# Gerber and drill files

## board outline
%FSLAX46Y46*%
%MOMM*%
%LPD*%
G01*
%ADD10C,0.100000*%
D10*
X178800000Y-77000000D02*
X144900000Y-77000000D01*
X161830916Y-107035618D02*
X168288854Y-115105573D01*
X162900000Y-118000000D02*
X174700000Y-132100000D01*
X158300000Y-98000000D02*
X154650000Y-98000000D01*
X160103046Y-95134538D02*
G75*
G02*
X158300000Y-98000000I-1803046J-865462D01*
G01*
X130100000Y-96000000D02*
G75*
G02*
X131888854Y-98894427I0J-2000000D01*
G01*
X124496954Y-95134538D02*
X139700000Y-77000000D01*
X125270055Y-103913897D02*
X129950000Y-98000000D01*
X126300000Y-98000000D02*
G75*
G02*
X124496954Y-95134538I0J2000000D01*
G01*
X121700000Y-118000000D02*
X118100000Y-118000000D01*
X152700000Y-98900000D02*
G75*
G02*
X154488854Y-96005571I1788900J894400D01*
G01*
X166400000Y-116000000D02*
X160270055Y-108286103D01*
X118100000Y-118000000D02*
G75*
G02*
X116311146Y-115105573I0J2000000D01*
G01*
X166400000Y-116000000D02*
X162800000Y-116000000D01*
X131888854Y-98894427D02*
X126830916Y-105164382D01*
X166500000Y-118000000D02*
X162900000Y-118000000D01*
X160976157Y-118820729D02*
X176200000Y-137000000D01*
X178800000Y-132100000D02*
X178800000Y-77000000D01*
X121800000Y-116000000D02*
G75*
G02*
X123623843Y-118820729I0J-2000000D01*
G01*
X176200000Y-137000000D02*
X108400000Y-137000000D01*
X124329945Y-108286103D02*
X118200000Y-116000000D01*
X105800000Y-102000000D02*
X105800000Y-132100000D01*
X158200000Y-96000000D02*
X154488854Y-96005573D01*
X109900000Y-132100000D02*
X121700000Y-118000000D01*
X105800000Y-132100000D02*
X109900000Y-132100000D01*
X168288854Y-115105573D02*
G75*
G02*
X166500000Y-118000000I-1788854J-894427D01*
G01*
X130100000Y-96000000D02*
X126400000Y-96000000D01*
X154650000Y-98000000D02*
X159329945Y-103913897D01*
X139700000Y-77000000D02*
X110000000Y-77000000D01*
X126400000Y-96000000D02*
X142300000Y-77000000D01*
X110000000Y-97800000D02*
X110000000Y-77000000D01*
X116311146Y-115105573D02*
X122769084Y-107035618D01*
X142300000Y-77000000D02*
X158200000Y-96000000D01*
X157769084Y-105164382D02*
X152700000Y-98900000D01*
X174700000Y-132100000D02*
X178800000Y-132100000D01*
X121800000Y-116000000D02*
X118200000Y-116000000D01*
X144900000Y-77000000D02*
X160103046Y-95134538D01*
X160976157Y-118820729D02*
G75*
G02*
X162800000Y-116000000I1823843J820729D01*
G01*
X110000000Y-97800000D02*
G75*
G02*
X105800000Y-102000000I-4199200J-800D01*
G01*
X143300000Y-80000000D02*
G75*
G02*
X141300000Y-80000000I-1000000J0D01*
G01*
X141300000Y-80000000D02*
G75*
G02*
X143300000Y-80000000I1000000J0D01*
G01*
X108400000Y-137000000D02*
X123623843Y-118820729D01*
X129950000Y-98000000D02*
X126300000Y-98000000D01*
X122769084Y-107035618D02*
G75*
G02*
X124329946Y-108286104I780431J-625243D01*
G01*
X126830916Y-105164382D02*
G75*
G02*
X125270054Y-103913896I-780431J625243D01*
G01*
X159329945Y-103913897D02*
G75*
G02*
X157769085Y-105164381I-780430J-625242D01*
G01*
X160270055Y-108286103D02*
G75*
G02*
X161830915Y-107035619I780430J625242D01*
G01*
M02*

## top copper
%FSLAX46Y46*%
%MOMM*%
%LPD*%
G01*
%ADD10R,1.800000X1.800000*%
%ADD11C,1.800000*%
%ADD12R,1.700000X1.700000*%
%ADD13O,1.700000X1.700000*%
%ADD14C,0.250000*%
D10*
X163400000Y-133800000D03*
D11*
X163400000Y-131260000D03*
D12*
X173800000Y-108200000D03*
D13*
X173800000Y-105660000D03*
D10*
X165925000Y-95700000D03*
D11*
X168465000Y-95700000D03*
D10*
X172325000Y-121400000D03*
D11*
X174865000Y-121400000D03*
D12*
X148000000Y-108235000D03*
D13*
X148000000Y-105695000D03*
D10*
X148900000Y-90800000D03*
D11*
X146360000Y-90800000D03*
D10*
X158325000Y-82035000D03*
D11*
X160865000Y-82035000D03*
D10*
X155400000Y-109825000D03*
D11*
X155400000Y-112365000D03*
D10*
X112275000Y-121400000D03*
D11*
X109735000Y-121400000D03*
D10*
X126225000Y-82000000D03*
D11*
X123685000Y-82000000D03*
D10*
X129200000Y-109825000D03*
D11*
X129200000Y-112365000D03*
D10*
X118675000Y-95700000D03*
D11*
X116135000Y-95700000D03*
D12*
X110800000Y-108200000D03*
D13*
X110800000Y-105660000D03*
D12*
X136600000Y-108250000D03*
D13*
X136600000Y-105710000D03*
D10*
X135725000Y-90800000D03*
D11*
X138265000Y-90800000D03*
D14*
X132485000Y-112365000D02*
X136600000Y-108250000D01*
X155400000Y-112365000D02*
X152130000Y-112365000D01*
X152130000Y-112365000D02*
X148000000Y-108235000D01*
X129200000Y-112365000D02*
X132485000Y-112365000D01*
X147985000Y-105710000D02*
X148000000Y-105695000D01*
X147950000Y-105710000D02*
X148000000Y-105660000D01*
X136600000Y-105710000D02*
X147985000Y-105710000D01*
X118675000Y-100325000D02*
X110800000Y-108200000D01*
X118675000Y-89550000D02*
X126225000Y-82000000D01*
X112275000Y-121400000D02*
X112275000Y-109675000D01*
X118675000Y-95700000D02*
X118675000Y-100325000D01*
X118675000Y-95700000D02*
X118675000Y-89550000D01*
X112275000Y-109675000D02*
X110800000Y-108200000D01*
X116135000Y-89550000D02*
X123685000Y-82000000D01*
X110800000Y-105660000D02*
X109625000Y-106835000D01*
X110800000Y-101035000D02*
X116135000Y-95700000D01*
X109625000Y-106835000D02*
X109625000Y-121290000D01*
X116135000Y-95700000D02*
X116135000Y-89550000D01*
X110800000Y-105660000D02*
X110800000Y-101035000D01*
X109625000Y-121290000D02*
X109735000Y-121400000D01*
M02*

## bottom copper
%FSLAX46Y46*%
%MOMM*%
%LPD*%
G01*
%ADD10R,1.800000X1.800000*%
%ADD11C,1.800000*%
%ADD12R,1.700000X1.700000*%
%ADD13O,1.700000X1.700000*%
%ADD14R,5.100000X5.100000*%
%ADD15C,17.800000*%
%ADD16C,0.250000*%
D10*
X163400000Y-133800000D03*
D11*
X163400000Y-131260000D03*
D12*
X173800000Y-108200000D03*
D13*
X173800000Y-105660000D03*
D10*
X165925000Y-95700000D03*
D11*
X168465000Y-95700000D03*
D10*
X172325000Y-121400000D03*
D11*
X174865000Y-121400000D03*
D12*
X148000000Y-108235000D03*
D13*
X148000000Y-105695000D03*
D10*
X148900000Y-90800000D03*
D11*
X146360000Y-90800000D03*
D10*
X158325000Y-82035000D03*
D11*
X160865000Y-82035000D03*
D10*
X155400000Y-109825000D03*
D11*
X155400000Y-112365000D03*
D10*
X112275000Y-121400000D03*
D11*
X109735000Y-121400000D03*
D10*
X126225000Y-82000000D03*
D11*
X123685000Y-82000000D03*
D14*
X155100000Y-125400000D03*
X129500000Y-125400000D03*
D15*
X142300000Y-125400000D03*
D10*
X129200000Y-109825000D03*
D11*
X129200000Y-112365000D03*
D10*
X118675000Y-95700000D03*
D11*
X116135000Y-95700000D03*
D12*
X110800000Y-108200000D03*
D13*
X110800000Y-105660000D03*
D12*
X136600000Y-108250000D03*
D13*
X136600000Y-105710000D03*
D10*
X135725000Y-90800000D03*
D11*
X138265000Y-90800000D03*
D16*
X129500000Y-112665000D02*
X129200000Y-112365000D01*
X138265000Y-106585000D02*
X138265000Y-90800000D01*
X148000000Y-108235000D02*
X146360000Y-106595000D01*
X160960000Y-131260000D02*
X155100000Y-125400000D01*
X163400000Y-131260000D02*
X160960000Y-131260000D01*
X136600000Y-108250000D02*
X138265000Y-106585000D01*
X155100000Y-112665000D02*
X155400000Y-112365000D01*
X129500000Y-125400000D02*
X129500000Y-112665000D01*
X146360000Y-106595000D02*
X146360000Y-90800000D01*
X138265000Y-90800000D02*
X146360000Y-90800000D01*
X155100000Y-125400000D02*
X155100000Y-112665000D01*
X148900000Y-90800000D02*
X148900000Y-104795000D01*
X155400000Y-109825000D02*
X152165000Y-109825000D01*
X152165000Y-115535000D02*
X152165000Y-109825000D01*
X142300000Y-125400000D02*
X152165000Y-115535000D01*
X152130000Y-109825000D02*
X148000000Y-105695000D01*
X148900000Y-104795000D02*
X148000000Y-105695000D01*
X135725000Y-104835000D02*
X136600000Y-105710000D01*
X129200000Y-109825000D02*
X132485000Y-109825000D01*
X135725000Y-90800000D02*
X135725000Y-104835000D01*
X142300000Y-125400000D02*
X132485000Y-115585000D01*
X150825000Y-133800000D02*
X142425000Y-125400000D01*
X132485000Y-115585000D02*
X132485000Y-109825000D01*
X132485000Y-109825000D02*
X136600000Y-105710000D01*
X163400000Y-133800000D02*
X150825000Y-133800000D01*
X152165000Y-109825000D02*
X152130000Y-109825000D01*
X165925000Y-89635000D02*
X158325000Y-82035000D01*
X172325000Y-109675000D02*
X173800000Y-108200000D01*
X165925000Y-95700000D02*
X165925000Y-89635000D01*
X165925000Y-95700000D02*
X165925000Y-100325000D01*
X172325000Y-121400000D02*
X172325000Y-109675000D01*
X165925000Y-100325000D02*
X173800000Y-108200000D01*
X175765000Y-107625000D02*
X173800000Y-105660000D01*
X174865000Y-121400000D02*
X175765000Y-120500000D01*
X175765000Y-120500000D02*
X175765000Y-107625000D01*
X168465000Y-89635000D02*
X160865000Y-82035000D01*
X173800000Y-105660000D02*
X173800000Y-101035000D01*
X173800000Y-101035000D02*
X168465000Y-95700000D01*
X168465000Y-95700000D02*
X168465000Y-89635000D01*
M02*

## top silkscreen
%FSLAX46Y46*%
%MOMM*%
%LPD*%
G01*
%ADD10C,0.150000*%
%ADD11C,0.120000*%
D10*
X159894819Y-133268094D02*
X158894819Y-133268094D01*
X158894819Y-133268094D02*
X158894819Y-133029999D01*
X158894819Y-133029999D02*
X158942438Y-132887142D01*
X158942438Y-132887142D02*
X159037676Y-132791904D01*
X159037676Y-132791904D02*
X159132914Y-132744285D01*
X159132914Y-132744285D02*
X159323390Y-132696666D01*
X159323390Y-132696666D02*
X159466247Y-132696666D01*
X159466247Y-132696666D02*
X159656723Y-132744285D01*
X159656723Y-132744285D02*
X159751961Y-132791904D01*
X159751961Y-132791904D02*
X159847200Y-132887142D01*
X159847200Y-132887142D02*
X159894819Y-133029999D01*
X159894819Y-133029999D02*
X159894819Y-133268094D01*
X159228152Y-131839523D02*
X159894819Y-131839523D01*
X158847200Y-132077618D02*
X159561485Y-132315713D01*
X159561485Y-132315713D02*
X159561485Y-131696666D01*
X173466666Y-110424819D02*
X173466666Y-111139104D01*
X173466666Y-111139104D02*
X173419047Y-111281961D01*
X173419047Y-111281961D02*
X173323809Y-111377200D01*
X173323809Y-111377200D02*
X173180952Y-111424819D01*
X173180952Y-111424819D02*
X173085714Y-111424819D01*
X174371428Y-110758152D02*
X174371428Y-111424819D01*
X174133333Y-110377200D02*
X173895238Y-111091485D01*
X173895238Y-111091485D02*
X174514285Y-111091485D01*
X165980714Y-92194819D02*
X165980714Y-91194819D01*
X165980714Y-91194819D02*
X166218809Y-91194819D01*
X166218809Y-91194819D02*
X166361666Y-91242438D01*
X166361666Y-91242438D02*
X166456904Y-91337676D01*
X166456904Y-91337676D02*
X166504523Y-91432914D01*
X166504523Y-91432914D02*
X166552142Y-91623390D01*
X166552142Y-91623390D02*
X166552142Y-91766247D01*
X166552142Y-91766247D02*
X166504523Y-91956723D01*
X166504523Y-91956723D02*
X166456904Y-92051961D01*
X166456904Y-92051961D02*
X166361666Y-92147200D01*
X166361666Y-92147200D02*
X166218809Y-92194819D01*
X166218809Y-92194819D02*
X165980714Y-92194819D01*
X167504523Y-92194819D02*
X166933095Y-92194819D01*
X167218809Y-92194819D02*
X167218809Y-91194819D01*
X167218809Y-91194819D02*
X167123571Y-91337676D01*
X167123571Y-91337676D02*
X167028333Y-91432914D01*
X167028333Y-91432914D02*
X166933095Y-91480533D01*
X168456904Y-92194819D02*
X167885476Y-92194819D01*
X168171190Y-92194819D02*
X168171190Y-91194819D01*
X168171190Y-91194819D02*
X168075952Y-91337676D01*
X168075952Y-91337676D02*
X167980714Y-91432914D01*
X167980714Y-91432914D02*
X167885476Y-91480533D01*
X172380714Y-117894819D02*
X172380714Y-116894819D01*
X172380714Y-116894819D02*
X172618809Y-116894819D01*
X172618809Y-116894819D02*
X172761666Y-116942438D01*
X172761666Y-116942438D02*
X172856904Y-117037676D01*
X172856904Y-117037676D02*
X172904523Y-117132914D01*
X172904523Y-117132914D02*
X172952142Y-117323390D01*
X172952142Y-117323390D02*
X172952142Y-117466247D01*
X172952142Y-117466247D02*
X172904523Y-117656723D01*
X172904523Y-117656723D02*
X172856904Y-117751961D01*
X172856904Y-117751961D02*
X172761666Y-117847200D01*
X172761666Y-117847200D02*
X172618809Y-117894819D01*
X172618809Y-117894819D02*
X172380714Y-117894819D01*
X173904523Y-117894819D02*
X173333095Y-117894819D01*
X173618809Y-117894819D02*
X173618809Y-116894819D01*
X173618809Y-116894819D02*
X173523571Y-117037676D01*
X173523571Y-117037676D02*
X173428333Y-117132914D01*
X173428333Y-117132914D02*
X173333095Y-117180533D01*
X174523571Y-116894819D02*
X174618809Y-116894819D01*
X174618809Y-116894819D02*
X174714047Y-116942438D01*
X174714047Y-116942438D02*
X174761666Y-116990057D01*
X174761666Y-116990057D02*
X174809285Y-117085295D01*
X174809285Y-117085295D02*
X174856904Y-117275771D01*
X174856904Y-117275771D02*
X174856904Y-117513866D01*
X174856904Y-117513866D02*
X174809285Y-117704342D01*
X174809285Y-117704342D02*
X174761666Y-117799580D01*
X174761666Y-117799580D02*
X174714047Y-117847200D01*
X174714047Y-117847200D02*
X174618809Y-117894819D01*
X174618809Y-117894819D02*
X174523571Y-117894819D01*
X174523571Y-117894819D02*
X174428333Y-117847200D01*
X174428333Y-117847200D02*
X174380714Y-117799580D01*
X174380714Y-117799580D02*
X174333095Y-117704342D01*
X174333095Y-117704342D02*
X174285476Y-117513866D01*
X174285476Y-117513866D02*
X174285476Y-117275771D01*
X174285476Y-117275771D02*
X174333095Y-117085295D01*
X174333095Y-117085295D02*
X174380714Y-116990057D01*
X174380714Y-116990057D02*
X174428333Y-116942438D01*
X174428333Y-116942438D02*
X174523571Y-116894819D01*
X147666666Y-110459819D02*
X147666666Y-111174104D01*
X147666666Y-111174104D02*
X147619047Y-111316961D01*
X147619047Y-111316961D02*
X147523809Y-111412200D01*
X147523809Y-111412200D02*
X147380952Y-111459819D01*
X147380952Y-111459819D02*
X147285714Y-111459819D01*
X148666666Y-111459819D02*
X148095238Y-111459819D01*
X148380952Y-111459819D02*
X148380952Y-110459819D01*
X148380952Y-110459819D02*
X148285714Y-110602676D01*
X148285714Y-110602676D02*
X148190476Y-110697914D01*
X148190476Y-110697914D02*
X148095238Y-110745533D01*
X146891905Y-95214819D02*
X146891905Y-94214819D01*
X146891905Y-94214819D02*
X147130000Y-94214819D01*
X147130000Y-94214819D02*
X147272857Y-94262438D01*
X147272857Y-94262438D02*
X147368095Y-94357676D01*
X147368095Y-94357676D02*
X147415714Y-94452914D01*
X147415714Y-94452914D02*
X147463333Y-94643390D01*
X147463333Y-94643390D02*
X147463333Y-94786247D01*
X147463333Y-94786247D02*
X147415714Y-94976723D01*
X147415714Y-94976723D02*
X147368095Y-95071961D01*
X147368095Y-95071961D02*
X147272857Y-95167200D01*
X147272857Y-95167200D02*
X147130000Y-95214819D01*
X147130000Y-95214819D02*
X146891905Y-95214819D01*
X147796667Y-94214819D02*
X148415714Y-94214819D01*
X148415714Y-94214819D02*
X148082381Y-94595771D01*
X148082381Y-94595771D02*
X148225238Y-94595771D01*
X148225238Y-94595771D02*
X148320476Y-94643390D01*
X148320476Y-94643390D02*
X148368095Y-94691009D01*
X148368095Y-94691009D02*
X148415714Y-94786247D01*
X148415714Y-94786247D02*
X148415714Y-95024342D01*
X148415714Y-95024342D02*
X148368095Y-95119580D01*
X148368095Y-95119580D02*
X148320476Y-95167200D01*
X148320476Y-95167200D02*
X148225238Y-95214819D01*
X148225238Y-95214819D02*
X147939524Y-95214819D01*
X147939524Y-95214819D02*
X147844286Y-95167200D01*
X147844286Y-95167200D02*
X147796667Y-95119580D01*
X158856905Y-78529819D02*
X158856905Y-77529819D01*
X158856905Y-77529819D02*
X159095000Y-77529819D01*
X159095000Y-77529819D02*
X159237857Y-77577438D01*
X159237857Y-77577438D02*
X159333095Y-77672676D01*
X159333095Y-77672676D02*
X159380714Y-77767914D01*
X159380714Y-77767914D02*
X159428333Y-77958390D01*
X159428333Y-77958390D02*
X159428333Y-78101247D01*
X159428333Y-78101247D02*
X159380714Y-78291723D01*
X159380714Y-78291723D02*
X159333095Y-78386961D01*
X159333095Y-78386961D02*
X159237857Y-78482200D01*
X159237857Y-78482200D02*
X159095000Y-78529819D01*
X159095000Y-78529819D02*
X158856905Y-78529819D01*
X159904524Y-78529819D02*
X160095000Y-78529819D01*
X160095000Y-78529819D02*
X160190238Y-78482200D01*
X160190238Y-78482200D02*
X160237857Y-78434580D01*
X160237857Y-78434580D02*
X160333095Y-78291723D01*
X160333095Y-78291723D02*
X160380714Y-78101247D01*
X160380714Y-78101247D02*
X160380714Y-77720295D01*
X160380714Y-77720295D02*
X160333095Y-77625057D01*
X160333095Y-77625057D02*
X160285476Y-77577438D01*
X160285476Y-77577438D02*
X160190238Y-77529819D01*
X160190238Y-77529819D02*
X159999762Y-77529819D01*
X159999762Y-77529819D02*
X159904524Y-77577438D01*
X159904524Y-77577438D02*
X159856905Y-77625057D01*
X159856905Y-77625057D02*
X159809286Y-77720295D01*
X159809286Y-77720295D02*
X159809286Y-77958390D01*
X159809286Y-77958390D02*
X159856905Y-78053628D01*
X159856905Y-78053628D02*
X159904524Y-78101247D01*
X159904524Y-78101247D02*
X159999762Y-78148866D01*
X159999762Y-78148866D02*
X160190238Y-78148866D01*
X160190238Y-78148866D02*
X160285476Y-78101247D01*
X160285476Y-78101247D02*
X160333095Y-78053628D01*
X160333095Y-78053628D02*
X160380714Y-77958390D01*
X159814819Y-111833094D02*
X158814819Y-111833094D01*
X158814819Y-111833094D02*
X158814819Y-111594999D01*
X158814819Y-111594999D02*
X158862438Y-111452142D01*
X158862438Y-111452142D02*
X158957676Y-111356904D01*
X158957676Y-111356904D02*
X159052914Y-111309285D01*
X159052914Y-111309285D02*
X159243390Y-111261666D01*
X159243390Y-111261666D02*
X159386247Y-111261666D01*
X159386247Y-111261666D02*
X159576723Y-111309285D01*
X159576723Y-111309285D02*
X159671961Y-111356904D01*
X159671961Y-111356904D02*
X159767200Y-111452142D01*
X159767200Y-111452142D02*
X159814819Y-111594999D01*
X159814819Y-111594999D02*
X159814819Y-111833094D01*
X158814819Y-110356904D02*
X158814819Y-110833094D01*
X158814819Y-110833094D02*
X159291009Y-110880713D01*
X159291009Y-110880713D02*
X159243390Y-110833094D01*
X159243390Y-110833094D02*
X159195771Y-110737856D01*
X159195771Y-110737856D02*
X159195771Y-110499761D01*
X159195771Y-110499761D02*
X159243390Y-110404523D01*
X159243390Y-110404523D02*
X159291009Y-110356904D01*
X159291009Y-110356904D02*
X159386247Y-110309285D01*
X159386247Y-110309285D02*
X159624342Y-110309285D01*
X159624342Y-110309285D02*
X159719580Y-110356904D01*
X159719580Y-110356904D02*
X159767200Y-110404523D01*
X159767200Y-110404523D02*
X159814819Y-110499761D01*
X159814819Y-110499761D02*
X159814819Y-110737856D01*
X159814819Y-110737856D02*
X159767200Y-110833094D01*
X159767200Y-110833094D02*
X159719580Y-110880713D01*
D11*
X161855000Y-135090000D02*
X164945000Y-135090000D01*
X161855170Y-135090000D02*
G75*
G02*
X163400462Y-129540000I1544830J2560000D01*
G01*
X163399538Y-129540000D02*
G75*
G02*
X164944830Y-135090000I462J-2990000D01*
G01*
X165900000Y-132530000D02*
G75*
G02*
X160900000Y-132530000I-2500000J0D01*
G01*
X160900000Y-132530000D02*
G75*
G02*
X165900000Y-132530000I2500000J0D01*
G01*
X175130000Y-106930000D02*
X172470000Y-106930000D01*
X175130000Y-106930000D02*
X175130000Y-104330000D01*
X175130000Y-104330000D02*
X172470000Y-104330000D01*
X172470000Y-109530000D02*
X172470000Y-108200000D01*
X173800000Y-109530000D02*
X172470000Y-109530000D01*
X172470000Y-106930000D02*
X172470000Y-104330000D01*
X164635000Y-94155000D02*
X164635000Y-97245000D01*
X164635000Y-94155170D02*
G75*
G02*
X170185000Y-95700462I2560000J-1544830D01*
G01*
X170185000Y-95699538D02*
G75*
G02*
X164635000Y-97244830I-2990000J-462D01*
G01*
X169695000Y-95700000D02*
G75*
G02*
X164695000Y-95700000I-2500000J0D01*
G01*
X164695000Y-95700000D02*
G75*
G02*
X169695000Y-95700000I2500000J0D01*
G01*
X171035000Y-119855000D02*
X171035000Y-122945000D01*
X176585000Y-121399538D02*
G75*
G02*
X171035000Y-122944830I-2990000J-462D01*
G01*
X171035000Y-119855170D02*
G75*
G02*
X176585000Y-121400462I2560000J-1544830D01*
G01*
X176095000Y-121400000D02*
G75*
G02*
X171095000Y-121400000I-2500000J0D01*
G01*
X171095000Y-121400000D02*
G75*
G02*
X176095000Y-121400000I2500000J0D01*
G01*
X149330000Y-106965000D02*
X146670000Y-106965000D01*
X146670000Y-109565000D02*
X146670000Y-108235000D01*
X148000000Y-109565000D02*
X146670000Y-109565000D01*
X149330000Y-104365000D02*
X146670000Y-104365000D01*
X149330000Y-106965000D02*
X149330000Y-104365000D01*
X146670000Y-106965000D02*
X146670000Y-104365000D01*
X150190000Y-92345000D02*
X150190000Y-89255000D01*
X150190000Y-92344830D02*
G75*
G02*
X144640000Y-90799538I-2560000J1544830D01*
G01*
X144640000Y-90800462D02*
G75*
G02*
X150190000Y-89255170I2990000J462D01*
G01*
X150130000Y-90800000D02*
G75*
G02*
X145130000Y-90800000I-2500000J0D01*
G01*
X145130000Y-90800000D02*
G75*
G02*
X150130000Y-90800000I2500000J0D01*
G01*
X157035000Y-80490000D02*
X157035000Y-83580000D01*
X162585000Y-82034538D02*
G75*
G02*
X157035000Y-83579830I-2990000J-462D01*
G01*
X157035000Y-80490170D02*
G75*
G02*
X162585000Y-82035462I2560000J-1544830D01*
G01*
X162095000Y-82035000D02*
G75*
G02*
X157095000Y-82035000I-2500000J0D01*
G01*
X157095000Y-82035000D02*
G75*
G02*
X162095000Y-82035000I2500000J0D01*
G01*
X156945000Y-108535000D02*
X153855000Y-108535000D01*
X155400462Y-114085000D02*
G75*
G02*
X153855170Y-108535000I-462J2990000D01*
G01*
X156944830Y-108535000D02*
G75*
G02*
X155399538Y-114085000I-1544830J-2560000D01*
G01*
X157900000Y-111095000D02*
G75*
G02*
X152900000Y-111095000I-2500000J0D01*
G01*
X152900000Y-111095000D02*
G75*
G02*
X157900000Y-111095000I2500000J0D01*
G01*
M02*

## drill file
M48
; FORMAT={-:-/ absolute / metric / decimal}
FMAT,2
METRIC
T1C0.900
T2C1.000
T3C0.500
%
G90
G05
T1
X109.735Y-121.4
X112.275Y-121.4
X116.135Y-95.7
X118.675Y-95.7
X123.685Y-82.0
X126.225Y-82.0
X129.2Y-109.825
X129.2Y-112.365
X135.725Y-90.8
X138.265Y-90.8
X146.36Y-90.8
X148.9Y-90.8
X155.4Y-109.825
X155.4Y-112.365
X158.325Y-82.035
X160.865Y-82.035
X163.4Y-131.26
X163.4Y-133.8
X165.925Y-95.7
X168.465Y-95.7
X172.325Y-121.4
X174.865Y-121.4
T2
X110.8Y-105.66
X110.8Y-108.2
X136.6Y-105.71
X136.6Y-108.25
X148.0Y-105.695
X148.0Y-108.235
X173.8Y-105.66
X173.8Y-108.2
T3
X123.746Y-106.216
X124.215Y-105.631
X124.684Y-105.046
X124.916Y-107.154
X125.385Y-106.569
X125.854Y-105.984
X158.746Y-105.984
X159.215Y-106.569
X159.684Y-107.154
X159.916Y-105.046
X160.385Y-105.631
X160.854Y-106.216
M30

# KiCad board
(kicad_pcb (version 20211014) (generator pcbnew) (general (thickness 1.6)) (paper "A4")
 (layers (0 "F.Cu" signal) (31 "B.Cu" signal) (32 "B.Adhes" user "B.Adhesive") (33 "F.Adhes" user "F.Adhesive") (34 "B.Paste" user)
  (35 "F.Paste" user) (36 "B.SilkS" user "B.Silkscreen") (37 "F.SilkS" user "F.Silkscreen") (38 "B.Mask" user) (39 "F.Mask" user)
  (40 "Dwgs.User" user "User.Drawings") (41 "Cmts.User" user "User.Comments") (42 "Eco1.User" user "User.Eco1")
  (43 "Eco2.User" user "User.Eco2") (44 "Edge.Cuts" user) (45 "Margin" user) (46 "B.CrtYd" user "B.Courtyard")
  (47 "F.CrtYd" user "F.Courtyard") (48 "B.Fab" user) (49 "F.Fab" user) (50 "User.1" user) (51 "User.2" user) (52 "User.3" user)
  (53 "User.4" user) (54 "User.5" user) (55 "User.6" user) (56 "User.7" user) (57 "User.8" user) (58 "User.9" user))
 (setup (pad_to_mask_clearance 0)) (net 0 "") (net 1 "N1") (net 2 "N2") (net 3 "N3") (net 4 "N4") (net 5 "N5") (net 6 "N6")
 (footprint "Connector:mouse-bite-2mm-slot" (layer "F.Cu") (at 124.8 106.1 -128.7)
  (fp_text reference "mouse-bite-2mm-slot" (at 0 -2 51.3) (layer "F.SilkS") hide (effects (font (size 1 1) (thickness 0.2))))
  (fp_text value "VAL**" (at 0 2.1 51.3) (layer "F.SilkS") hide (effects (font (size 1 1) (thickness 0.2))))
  (fp_arc (start 2 1) (mid 1 0) (end 2 -1) (layer "Edge.Cuts") (width 0.1))
  (fp_arc (start -2 -1) (mid -1 0) (end -2 1) (layer "Edge.Cuts") (width 0.1))
  (pad "" np_thru_hole circle (at 0.75 0.75 231.3) (size 0.5 0.5) (drill 0.5) (layers F&B.Cu *.Mask))
  (pad "" np_thru_hole circle (at 0.75 -0.75 231.3) (size 0.5 0.5) (drill 0.5) (layers F&B.Cu *.Mask))
  (pad "" np_thru_hole circle (at 0 0.75 231.3) (size 0.5 0.5) (drill 0.5) (layers F&B.Cu *.Mask))
  (pad "" np_thru_hole circle (at 0 -0.75 231.3) (size 0.5 0.5) (drill 0.5) (layers F&B.Cu *.Mask))
  (pad "" np_thru_hole circle (at -0.75 0.75 231.3) (size 0.5 0.5) (drill 0.5) (layers F&B.Cu *.Mask))
  (pad "" np_thru_hole circle (at -0.75 -0.75 231.3) (size 0.5 0.5) (drill 0.5) (layers F&B.Cu *.Mask)))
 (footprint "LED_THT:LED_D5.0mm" (layer "F.Cu") (at 163.4 133.8 90)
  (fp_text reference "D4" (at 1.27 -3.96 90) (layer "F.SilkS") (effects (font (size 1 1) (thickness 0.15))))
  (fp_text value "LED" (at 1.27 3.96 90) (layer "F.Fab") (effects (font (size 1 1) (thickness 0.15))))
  (fp_line (start -1.29 -1.545) (end -1.29 1.545) (layer "F.SilkS") (width 0.12))
  (fp_arc (start -1.29 -1.54483) (mid 2.072002 -2.880433) (end 4.26 0.000462) (layer "F.SilkS") (width 0.12))
  (fp_arc (start 4.26 -0.000462) (mid 2.072002 2.880433) (end -1.29 1.54483) (layer "F.SilkS") (width 0.12))
  (fp_circle (center 1.27 0) (end 3.77 0) (layer "F.SilkS") (width 0.12) (fill none))
  (pad "1" thru_hole rect (at 0 0 90) (size 1.8 1.8) (drill 0.9) (layers *.Cu *.Mask) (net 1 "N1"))
  (pad "2" thru_hole circle (at 2.54 0 90) (size 1.8 1.8) (drill 0.9) (layers *.Cu *.Mask) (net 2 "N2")))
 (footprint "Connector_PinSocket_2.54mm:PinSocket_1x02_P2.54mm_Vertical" (layer "F.Cu") (at 173.8 108.2 180)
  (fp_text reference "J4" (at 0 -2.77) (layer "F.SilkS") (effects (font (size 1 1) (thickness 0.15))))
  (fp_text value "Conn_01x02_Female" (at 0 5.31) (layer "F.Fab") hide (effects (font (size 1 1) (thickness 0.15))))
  (fp_line (start -1.33 1.27) (end 1.33 1.27) (layer "F.SilkS") (width 0.12))
  (fp_line (start -1.33 1.27) (end -1.33 3.87) (layer "F.SilkS") (width 0.12))
  (fp_line (start -1.33 3.87) (end 1.33 3.87) (layer "F.SilkS") (width 0.12))
  (fp_line (start 1.33 -1.33) (end 1.33 0) (layer "F.SilkS") (width 0.12))
  (fp_line (start 0 -1.33) (end 1.33 -1.33) (layer "F.SilkS") (width 0.12))
  (fp_line (start 1.33 1.27) (end 1.33 3.87) (layer "F.SilkS") (width 0.12))
  (pad "1" thru_hole rect (at 0 0 180) (size 1.7 1.7) (drill 1) (layers *.Cu *.Mask) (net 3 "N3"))
  (pad "2" thru_hole oval (at 0 2.54 180) (size 1.7 1.7) (drill 1) (layers *.Cu *.Mask) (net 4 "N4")))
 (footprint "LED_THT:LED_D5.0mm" (layer "F.Cu") (at 165.925 95.7)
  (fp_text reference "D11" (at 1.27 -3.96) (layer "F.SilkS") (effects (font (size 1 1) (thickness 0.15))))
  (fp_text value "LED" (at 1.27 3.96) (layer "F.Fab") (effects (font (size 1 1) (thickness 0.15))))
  (fp_line (start -1.29 -1.545) (end -1.29 1.545) (layer "F.SilkS") (width 0.12))
  (fp_arc (start -1.29 -1.54483) (mid 2.072002 -2.880433) (end 4.26 0.000462) (layer "F.SilkS") (width 0.12))
  (fp_arc (start 4.26 -0.000462) (mid 2.072002 2.880433) (end -1.29 1.54483) (layer "F.SilkS") (width 0.12))
  (fp_circle (center 1.27 0) (end 3.77 0) (layer "F.SilkS") (width 0.12) (fill none))
  (pad "1" thru_hole rect (at 0 0) (size 1.8 1.8) (drill 0.9) (layers *.Cu *.Mask) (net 3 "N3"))
  (pad "2" thru_hole circle (at 2.54 0) (size 1.8 1.8) (drill 0.9) (layers *.Cu *.Mask) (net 4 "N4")))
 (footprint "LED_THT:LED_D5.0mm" (layer "F.Cu") (at 172.325 121.4)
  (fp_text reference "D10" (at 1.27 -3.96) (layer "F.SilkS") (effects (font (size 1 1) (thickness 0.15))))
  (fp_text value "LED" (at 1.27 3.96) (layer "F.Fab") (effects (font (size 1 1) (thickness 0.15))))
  (fp_line (start -1.29 -1.545) (end -1.29 1.545) (layer "F.SilkS") (width 0.12))
  (fp_arc (start 4.26 -0.000462) (mid 2.072002 2.880433) (end -1.29 1.54483) (layer "F.SilkS") (width 0.12))
  (fp_arc (start -1.29 -1.54483) (mid 2.072002 -2.880433) (end 4.26 0.000462) (layer "F.SilkS") (width 0.12))
  (fp_circle (center 1.27 0) (end 3.77 0) (layer "F.SilkS") (width 0.12) (fill none))
  (pad "1" thru_hole rect (at 0 0) (size 1.8 1.8) (drill 0.9) (layers *.Cu *.Mask) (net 3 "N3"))
  (pad "2" thru_hole circle (at 2.54 0) (size 1.8 1.8) (drill 0.9) (layers *.Cu *.Mask) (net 4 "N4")))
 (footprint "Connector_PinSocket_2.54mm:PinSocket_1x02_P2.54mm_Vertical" (layer "F.Cu") (at 148 108.235 180)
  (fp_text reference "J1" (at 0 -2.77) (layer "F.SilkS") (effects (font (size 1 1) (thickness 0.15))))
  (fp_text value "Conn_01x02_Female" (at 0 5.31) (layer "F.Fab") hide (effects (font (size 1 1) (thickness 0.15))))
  (fp_line (start -1.33 1.27) (end 1.33 1.27) (layer "F.SilkS") (width 0.12))
  (fp_line (start 1.33 -1.33) (end 1.33 0) (layer "F.SilkS") (width 0.12))
  (fp_line (start 0 -1.33) (end 1.33 -1.33) (layer "F.SilkS") (width 0.12))
  (fp_line (start -1.33 3.87) (end 1.33 3.87) (layer "F.SilkS") (width 0.12))
  (fp_line (start -1.33 1.27) (end -1.33 3.87) (layer "F.SilkS") (width 0.12))
  (fp_line (start 1.33 1.27) (end 1.33 3.87) (layer "F.SilkS") (width 0.12))
  (pad "1" thru_hole rect (at 0 0 180) (size 1.7 1.7) (drill 1) (layers *.Cu *.Mask) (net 2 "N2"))
  (pad "2" thru_hole oval (at 0 2.54 180) (size 1.7 1.7) (drill 1) (layers *.Cu *.Mask) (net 1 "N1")))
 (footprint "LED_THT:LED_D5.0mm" (layer "F.Cu") (at 148.9 90.8 180)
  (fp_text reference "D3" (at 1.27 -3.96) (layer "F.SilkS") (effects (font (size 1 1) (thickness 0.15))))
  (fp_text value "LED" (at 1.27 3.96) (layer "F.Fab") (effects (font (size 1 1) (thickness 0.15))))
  (fp_line (start -1.29 -1.545) (end -1.29 1.545) (layer "F.SilkS") (width 0.12))
  (fp_arc (start -1.29 -1.54483) (mid 2.072002 -2.880433) (end 4.26 0.000462) (layer "F.SilkS") (width 0.12))
  (fp_arc (start 4.26 -0.000462) (mid 2.072002 2.880433) (end -1.29 1.54483) (layer "F.SilkS") (width 0.12))
  (fp_circle (center 1.27 0) (end 3.77 0) (layer "F.SilkS") (width 0.12) (fill none))
  (pad "1" thru_hole rect (at 0 0 180) (size 1.8 1.8) (drill 0.9) (layers *.Cu *.Mask) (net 1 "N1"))
  (pad "2" thru_hole circle (at 2.54 0 180) (size 1.8 1.8) (drill 0.9) (layers *.Cu *.Mask) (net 2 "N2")))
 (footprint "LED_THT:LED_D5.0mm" (layer "F.Cu") (at 158.325 82.035)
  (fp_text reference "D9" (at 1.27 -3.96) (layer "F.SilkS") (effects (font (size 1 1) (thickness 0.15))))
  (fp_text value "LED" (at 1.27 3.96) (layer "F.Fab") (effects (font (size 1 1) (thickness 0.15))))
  (fp_line (start -1.29 -1.545) (end -1.29 1.545) (layer "F.SilkS") (width 0.12))
  (fp_arc (start 4.26 -0.000462) (mid 2.072002 2.880433) (end -1.29 1.54483) (layer "F.SilkS") (width 0.12))
  (fp_arc (start -1.29 -1.54483) (mid 2.072002 -2.880433) (end 4.26 0.000462) (layer "F.SilkS") (width 0.12))
  (fp_circle (center 1.27 0) (end 3.77 0) (layer "F.SilkS") (width 0.12) (fill none))
  (pad "1" thru_hole rect (at 0 0) (size 1.8 1.8) (drill 0.9) (layers *.Cu *.Mask) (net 3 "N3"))
  (pad "2" thru_hole circle (at 2.54 0) (size 1.8 1.8) (drill 0.9) (layers *.Cu *.Mask) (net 4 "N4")))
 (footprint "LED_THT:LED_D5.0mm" (layer "F.Cu") (at 155.4 109.825 -90)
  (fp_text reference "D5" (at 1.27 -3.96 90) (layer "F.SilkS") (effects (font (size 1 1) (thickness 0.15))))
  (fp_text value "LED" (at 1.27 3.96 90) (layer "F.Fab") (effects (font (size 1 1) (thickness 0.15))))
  (fp_line (start -1.29 -1.545) (end -1.29 1.545) (layer "F.SilkS") (width 0.12))
  (fp_arc (start 4.26 -0.000462) (mid 2.072002 2.880433) (end -1.29 1.54483) (layer "F.SilkS") (width 0.12))
  (fp_arc (start -1.29 -1.54483) (mid 2.072002 -2.880433) (end 4.26 0.000462) (layer "F.SilkS") (width 0.12))
  (fp_circle (center 1.27 0) (end 3.77 0) (layer "F.SilkS") (width 0.12) (fill none))
  (pad "1" thru_hole rect (at 0 0 270) (size 1.8 1.8) (drill 0.9) (layers *.Cu *.Mask) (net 1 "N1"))
  (pad "2" thru_hole circle (at 2.54 0 270) (size 1.8 1.8) (drill 0.9) (layers *.Cu *.Mask) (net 2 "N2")))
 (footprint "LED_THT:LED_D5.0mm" (layer "B.Cu") (at 112.275 121.4 180)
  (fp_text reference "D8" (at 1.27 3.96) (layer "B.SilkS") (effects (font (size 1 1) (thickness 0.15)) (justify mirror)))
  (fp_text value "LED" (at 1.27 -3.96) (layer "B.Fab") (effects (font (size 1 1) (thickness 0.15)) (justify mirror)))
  (pad "1" thru_hole rect (at 0 0 180) (size 1.8 1.8) (drill 0.9) (layers *.Cu *.Mask) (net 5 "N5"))
  (pad "2" thru_hole circle (at 2.54 0 180) (size 1.8 1.8) (drill 0.9) (layers *.Cu *.Mask) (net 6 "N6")))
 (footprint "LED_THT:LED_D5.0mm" (layer "B.Cu") (at 126.225 82 180)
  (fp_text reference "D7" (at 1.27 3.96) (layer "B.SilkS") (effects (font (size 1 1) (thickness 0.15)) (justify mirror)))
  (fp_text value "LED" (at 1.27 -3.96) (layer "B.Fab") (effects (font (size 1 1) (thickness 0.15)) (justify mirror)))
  (pad "1" thru_hole rect (at 0 0 180) (size 1.8 1.8) (drill 0.9) (layers *.Cu *.Mask) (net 5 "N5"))
  (pad "2" thru_hole circle (at 2.54 0 180) (size 1.8 1.8) (drill 0.9) (layers *.Cu *.Mask) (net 6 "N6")))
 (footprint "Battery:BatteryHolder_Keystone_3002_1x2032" (layer "B.Cu") (at 142.3 125.4)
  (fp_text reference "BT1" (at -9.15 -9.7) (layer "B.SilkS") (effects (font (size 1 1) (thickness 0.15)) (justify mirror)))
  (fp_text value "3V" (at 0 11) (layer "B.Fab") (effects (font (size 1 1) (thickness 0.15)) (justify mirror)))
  (pad "1" smd rect (at 12.8 0) (size 5.1 5.1) (layers "B.Cu" "B.Paste" "B.Mask") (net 2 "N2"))
  (pad "1" smd rect (at -12.8 0) (size 5.1 5.1) (layers "B.Cu" "B.Paste" "B.Mask") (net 2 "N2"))
  (pad "2" smd circle (at 0 0) (size 17.8 17.8) (layers "B.Cu" "B.Mask") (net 1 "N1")))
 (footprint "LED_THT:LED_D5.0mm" (layer "B.Cu") (at 129.2 109.825 -90)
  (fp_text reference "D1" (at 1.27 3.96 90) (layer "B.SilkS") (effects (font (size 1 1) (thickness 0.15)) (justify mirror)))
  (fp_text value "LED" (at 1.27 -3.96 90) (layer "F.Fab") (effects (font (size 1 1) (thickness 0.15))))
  (pad "1" thru_hole rect (at 0 0 270) (size 1.8 1.8) (drill 0.9) (layers *.Cu *.Mask) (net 1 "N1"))
  (pad "2" thru_hole circle (at 2.54 0 270) (size 1.8 1.8) (drill 0.9) (layers *.Cu *.Mask) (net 2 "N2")))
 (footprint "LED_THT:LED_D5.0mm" (layer "B.Cu") (at 118.675 95.7 180)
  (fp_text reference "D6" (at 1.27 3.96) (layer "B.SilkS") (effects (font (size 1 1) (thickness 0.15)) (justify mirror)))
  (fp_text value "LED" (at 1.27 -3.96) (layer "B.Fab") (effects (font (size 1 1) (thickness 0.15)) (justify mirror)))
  (pad "1" thru_hole rect (at 0 0 180) (size 1.8 1.8) (drill 0.9) (layers *.Cu *.Mask) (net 5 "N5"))
  (pad "2" thru_hole circle (at 2.54 0 180) (size 1.8 1.8) (drill 0.9) (layers *.Cu *.Mask) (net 6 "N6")))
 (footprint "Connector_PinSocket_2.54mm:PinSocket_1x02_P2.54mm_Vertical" (layer "B.Cu") (at 110.8 108.2)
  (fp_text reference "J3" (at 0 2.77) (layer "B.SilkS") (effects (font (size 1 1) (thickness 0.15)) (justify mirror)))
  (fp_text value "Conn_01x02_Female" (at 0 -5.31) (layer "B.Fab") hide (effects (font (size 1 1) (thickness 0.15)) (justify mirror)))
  (pad "1" thru_hole rect locked (at 0 0) (size 1.7 1.7) (drill 1) (layers *.Cu *.Mask) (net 5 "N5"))
  (pad "2" thru_hole oval (at 0 -2.54) (size 1.7 1.7) (drill 1) (layers *.Cu *.Mask) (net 6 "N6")))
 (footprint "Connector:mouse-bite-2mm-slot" (layer "B.Cu") (at 159.8 106.1 -51.3)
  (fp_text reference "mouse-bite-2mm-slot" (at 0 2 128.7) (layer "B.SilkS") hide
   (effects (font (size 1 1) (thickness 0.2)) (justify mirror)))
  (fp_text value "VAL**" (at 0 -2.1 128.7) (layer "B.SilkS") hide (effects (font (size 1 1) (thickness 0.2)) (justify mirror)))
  (fp_arc (start -2 -1) (mid -1 0) (end -2 1) (layer "Edge.Cuts") (width 0.1))
  (fp_arc (start 2 1) (mid 1 0) (end 2 -1) (layer "Edge.Cuts") (width 0.1))
  (pad "" np_thru_hole circle (at 0.75 -0.75 308.7) (size 0.5 0.5) (drill 0.5) (layers *.Cu *.Mask))
  (pad "" np_thru_hole circle (at 0 0.75 308.7) (size 0.5 0.5) (drill 0.5) (layers *.Cu *.Mask))
  (pad "" np_thru_hole circle (at -0.75 0.75 308.7) (size 0.5 0.5) (drill 0.5) (layers *.Cu *.Mask))
  (pad "" np_thru_hole circle (at 0 -0.75 308.7) (size 0.5 0.5) (drill 0.5) (layers *.Cu *.Mask))
  (pad "" np_thru_hole circle (at 0.75 0.75 308.7) (size 0.5 0.5) (drill 0.5) (layers *.Cu *.Mask))
  (pad "" np_thru_hole circle (at -0.75 -0.75 308.7) (size 0.5 0.5) (drill 0.5) (layers *.Cu *.Mask)))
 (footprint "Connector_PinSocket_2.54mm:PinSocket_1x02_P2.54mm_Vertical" (layer "B.Cu") (at 136.6 108.25)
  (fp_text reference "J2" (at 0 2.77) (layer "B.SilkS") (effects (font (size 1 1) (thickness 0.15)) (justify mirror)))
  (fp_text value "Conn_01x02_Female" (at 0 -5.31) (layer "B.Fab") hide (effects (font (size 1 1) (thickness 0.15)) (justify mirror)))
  (pad "1" thru_hole rect (at 0 0) (size 1.7 1.7) (drill 1) (layers *.Cu *.Mask) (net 2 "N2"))
  (pad "2" thru_hole oval (at 0 -2.54) (size 1.7 1.7) (drill 1) (layers *.Cu *.Mask) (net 1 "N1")))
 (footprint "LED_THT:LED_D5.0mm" (layer "B.Cu") (at 135.725 90.8)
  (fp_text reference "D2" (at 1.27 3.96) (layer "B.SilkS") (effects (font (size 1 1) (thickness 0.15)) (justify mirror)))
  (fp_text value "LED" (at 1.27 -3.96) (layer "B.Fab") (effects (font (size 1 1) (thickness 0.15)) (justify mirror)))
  (pad "1" thru_hole rect (at 0 0) (size 1.8 1.8) (drill 0.9) (layers *.Cu *.Mask) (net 1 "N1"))
  (pad "2" thru_hole circle (at 2.54 0) (size 1.8 1.8) (drill 0.9) (layers *.Cu *.Mask) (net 2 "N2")))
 (gr_line (start 178.8 77) (end 144.9 77) (layer "Edge.Cuts") (width 0.1))
 (gr_line (start 161.830916 107.035618) (end 168.288854 115.105573) (layer "Edge.Cuts") (width 0.1))
 (gr_line (start 162.9 118) (end 174.7 132.1) (layer "Edge.Cuts") (width 0.1))
 (gr_line (start 158.3 98) (end 154.65 98) (layer "Edge.Cuts") (width 0.1))
 (gr_arc (start 160.103046 95.134538) (mid 159.992767 97.065147) (end 158.3 98) (layer "Edge.Cuts") (width 0.1))
 (gr_arc (start 130.1 96) (mid 131.801302 96.948538) (end 131.888854 98.894427) (layer "Edge.Cuts") (width 0.1))
 (gr_line (start 124.496954 95.134538) (end 139.7 77) (layer "Edge.Cuts") (width 0.1))
 (gr_line (start 125.270055 103.913897) (end 129.95 98) (layer "Edge.Cuts") (width 0.1))
 (gr_arc (start 126.3 98) (mid 124.607232 97.065147) (end 124.496954 95.134538) (layer "Edge.Cuts") (width 0.1))
 (gr_line (start 121.7 118) (end 118.1 118) (layer "Edge.Cuts") (width 0.1))
 (gr_arc (start 152.7 98.9) (mid 152.787574 96.954123) (end 154.488854 96.005573) (layer "Edge.Cuts") (width 0.1))
 (gr_line (start 166.4 116) (end 160.270055 108.286103) (layer "Edge.Cuts") (width 0.1))
 (gr_arc (start 118.1 118) (mid 116.398698 117.051462) (end 116.311146 115.105573) (layer "Edge.Cuts") (width 0.1))
 (gr_line (start 166.4 116) (end 162.8 116) (layer "Edge.Cuts") (width 0.1))
 (gr_line (start 131.888854 98.894427) (end 126.830916 105.164382) (layer "Edge.Cuts") (width 0.1))
 (gr_line (start 166.5 118) (end 162.9 118) (layer "Edge.Cuts") (width 0.1))
 (gr_line (start 160.976157 118.820729) (end 176.2 137) (layer "Edge.Cuts") (width 0.1))
 (gr_line (start 178.8 132.1) (end 178.8 77) (layer "Edge.Cuts") (width 0.1))
 (gr_arc (start 121.8 116) (mid 123.479503 116.914058) (end 123.623843 118.820729) (layer "Edge.Cuts") (width 0.1))
 (gr_line (start 176.2 137) (end 108.4 137) (layer "Edge.Cuts") (width 0.1))
 (gr_line (start 124.329945 108.286103) (end 118.2 116) (layer "Edge.Cuts") (width 0.1))
 (gr_line (start 105.8 102) (end 105.8 132.1) (layer "Edge.Cuts") (width 0.1))
 (gr_line (start 158.2 96) (end 154.488854 96.005573) (layer "Edge.Cuts") (width 0.1))
 (gr_line (start 109.9 132.1) (end 121.7 118) (layer "Edge.Cuts") (width 0.1))
 (gr_line (start 105.8 132.1) (end 109.9 132.1) (layer "Edge.Cuts") (width 0.1))
 (gr_arc (start 168.288854 115.105573) (mid 168.201301 117.051462) (end 166.5 118) (layer "Edge.Cuts") (width 0.1))
 (gr_line (start 130.1 96) (end 126.4 96) (layer "Edge.Cuts") (width 0.1))
 (gr_line (start 154.65 98) (end 159.329945 103.913897) (layer "Edge.Cuts") (width 0.1))
 (gr_line (start 139.7 77) (end 110 77) (layer "Edge.Cuts") (width 0.1))
 (gr_line (start 126.4 96) (end 142.3 77) (layer "Edge.Cuts") (width 0.1))
 (gr_line (start 110 97.8) (end 110 77) (layer "Edge.Cuts") (width 0.1))
 (gr_line (start 116.311146 115.105573) (end 122.769084 107.035618) (layer "Edge.Cuts") (width 0.1))
 (gr_line (start 142.3 77) (end 158.2 96) (layer "Edge.Cuts") (width 0.1))
 (gr_line (start 157.769084 105.164382) (end 152.7 98.9) (layer "Edge.Cuts") (width 0.1))
 (gr_line (start 174.7 132.1) (end 178.8 132.1) (layer "Edge.Cuts") (width 0.1))
 (gr_line (start 121.8 116) (end 118.2 116) (layer "Edge.Cuts") (width 0.1))
 (gr_line (start 144.9 77) (end 160.103046 95.134538) (layer "Edge.Cuts") (width 0.1))
 (gr_arc (start 160.976157 118.820729) (mid 161.120498 116.914058) (end 162.8 116) (layer "Edge.Cuts") (width 0.1))
 (gr_arc (start 110 97.8) (mid 108.770083 100.770083) (end 105.8 102) (layer "Edge.Cuts") (width 0.1))
 (gr_circle (center 142.3 80) (end 142.3 81) (layer "Edge.Cuts") (width 0.1) (fill none))
 (gr_line (start 108.4 137) (end 123.623843 118.820729) (layer "Edge.Cuts") (width 0.1))
 (gr_line (start 129.95 98) (end 126.3 98) (layer "Edge.Cuts") (width 0.1))
 (segment (start 132.485 112.365) (end 136.6 108.25) (width 0.25) (layer "F.Cu") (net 2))
 (segment (start 155.4 112.365) (end 152.13 112.365) (width 0.25) (layer "F.Cu") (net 2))
 (segment (start 152.13 112.365) (end 148 108.235) (width 0.25) (layer "F.Cu") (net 2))
 (segment (start 129.2 112.365) (end 132.485 112.365) (width 0.25) (layer "F.Cu") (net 2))
 (segment (start 129.5 112.665) (end 129.2 112.365) (width 0.25) (layer "B.Cu") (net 2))
 (segment (start 138.265 106.585) (end 138.265 90.8) (width 0.25) (layer "B.Cu") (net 2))
 (segment (start 148 108.235) (end 146.36 106.595) (width 0.25) (layer "B.Cu") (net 2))
 (segment (start 160.96 131.26) (end 155.1 125.4) (width 0.25) (layer "B.Cu") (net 2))
 (segment (start 163.4 131.26) (end 160.96 131.26) (width 0.25) (layer "B.Cu") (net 2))
 (segment (start 136.6 108.25) (end 138.265 106.585) (width 0.25) (layer "B.Cu") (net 2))
 (segment (start 155.1 112.665) (end 155.4 112.365) (width 0.25) (layer "B.Cu") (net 2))
 (segment (start 129.5 125.4) (end 129.5 112.665) (width 0.25) (layer "B.Cu") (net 2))
 (segment (start 146.36 106.595) (end 146.36 90.8) (width 0.25) (layer "B.Cu") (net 2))
 (segment (start 138.265 90.8) (end 146.36 90.8) (width 0.25) (layer "B.Cu") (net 2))
 (segment (start 155.1 125.4) (end 155.1 112.665) (width 0.25) (layer "B.Cu") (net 2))
 (segment (start 147.985 105.71) (end 148 105.695) (width 0.25) (layer "F.Cu") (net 1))
 (segment (start 147.95 105.71) (end 148 105.66) (width 0.25) (layer "F.Cu") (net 1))
 (segment (start 136.6 105.71) (end 147.985 105.71) (width 0.25) (layer "F.Cu") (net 1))
 (segment (start 148.9 90.8) (end 148.9 104.795) (width 0.25) (layer "B.Cu") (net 1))
 (segment (start 155.4 109.825) (end 152.165 109.825) (width 0.25) (layer "B.Cu") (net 1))
 (segment (start 152.165 115.535) (end 152.165 109.825) (width 0.25) (layer "B.Cu") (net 1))
 (segment (start 142.3 125.4) (end 152.165 115.535) (width 0.25) (layer "B.Cu") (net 1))
 (segment (start 152.13 109.825) (end 148 105.695) (width 0.25) (layer "B.Cu") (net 1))
 (segment (start 148.9 104.795) (end 148 105.695) (width 0.25) (layer "B.Cu") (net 1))
 (segment (start 135.725 104.835) (end 136.6 105.71) (width 0.25) (layer "B.Cu") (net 1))
 (segment (start 129.2 109.825) (end 132.485 109.825) (width 0.25) (layer "B.Cu") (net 1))
 (segment (start 135.725 90.8) (end 135.725 104.835) (width 0.25) (layer "B.Cu") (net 1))
 (segment (start 142.3 125.4) (end 132.485 115.585) (width 0.25) (layer "B.Cu") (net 1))
 (segment (start 150.825 133.8) (end 142.425 125.4) (width 0.25) (layer "B.Cu") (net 1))
 (segment (start 132.485 115.585) (end 132.485 109.825) (width 0.25) (layer "B.Cu") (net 1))
 (segment (start 132.485 109.825) (end 136.6 105.71) (width 0.25) (layer "B.Cu") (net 1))
 (segment (start 163.4 133.8) (end 150.825 133.8) (width 0.25) (layer "B.Cu") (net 1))
 (segment (start 152.165 109.825) (end 152.13 109.825) (width 0.25) (layer "B.Cu") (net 1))
 (segment (start 118.675 100.325) (end 110.8 108.2) (width 0.25) (layer "F.Cu") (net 5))
 (segment (start 118.675 89.55) (end 126.225 82) (width 0.25) (layer "F.Cu") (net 5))
 (segment (start 112.275 121.4) (end 112.275 109.675) (width 0.25) (layer "F.Cu") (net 5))
 (segment (start 118.675 95.7) (end 118.675 100.325) (width 0.25) (layer "F.Cu") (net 5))
 (segment (start 118.675 95.7) (end 118.675 89.55) (width 0.25) (layer "F.Cu") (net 5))
 (segment (start 112.275 109.675) (end 110.8 108.2) (width 0.25) (layer "F.Cu") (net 5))
 (segment (start 116.135 89.55) (end 123.685 82) (width 0.25) (layer "F.Cu") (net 6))
 (segment (start 110.8 105.66) (end 109.625 106.835) (width 0.25) (layer "F.Cu") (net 6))
 (segment (start 110.8 101.035) (end 116.135 95.7) (width 0.25) (layer "F.Cu") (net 6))
 (segment (start 109.625 106.835) (end 109.625 121.29) (width 0.25) (layer "F.Cu") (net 6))
 (segment (start 116.135 95.7) (end 116.135 89.55) (width 0.25) (layer "F.Cu") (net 6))
 (segment (start 110.8 105.66) (end 110.8 101.035) (width 0.25) (layer "F.Cu") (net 6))
 (segment (start 109.625 121.29) (end 109.735 121.4) (width 0.25) (layer "F.Cu") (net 6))
 (segment (start 165.925 89.635) (end 158.325 82.035) (width 0.25) (layer "B.Cu") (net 3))
 (segment (start 172.325 109.675) (end 173.8 108.2) (width 0.25) (layer "B.Cu") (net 3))
 (segment (start 165.925 95.7) (end 165.925 89.635) (width 0.25) (layer "B.Cu") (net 3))
 (segment (start 165.925 95.7) (end 165.925 100.325) (width 0.25) (layer "B.Cu") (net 3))
 (segment (start 172.325 121.4) (end 172.325 109.675) (width 0.25) (layer "B.Cu") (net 3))
 (segment (start 165.925 100.325) (end 173.8 108.2) (width 0.25) (layer "B.Cu") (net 3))
 (segment (start 175.765 107.625) (end 173.8 105.66) (width 0.25) (layer "B.Cu") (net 4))
 (segment (start 174.865 121.4) (end 175.765 120.5) (width 0.25) (layer "B.Cu") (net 4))
 (segment (start 175.765 120.5) (end 175.765 107.625) (width 0.25) (layer "B.Cu") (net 4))
 (segment (start 168.465 89.635) (end 160.865 82.035) (width 0.25) (layer "B.Cu") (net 4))
 (segment (start 173.8 105.66) (end 173.8 101.035) (width 0.25) (layer "B.Cu") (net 4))
 (segment (start 173.8 101.035) (end 168.465 95.7) (width 0.25) (layer "B.Cu") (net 4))
 (segment (start 168.465 95.7) (end 168.465 89.635) (width 0.25) (layer "B.Cu") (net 4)))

